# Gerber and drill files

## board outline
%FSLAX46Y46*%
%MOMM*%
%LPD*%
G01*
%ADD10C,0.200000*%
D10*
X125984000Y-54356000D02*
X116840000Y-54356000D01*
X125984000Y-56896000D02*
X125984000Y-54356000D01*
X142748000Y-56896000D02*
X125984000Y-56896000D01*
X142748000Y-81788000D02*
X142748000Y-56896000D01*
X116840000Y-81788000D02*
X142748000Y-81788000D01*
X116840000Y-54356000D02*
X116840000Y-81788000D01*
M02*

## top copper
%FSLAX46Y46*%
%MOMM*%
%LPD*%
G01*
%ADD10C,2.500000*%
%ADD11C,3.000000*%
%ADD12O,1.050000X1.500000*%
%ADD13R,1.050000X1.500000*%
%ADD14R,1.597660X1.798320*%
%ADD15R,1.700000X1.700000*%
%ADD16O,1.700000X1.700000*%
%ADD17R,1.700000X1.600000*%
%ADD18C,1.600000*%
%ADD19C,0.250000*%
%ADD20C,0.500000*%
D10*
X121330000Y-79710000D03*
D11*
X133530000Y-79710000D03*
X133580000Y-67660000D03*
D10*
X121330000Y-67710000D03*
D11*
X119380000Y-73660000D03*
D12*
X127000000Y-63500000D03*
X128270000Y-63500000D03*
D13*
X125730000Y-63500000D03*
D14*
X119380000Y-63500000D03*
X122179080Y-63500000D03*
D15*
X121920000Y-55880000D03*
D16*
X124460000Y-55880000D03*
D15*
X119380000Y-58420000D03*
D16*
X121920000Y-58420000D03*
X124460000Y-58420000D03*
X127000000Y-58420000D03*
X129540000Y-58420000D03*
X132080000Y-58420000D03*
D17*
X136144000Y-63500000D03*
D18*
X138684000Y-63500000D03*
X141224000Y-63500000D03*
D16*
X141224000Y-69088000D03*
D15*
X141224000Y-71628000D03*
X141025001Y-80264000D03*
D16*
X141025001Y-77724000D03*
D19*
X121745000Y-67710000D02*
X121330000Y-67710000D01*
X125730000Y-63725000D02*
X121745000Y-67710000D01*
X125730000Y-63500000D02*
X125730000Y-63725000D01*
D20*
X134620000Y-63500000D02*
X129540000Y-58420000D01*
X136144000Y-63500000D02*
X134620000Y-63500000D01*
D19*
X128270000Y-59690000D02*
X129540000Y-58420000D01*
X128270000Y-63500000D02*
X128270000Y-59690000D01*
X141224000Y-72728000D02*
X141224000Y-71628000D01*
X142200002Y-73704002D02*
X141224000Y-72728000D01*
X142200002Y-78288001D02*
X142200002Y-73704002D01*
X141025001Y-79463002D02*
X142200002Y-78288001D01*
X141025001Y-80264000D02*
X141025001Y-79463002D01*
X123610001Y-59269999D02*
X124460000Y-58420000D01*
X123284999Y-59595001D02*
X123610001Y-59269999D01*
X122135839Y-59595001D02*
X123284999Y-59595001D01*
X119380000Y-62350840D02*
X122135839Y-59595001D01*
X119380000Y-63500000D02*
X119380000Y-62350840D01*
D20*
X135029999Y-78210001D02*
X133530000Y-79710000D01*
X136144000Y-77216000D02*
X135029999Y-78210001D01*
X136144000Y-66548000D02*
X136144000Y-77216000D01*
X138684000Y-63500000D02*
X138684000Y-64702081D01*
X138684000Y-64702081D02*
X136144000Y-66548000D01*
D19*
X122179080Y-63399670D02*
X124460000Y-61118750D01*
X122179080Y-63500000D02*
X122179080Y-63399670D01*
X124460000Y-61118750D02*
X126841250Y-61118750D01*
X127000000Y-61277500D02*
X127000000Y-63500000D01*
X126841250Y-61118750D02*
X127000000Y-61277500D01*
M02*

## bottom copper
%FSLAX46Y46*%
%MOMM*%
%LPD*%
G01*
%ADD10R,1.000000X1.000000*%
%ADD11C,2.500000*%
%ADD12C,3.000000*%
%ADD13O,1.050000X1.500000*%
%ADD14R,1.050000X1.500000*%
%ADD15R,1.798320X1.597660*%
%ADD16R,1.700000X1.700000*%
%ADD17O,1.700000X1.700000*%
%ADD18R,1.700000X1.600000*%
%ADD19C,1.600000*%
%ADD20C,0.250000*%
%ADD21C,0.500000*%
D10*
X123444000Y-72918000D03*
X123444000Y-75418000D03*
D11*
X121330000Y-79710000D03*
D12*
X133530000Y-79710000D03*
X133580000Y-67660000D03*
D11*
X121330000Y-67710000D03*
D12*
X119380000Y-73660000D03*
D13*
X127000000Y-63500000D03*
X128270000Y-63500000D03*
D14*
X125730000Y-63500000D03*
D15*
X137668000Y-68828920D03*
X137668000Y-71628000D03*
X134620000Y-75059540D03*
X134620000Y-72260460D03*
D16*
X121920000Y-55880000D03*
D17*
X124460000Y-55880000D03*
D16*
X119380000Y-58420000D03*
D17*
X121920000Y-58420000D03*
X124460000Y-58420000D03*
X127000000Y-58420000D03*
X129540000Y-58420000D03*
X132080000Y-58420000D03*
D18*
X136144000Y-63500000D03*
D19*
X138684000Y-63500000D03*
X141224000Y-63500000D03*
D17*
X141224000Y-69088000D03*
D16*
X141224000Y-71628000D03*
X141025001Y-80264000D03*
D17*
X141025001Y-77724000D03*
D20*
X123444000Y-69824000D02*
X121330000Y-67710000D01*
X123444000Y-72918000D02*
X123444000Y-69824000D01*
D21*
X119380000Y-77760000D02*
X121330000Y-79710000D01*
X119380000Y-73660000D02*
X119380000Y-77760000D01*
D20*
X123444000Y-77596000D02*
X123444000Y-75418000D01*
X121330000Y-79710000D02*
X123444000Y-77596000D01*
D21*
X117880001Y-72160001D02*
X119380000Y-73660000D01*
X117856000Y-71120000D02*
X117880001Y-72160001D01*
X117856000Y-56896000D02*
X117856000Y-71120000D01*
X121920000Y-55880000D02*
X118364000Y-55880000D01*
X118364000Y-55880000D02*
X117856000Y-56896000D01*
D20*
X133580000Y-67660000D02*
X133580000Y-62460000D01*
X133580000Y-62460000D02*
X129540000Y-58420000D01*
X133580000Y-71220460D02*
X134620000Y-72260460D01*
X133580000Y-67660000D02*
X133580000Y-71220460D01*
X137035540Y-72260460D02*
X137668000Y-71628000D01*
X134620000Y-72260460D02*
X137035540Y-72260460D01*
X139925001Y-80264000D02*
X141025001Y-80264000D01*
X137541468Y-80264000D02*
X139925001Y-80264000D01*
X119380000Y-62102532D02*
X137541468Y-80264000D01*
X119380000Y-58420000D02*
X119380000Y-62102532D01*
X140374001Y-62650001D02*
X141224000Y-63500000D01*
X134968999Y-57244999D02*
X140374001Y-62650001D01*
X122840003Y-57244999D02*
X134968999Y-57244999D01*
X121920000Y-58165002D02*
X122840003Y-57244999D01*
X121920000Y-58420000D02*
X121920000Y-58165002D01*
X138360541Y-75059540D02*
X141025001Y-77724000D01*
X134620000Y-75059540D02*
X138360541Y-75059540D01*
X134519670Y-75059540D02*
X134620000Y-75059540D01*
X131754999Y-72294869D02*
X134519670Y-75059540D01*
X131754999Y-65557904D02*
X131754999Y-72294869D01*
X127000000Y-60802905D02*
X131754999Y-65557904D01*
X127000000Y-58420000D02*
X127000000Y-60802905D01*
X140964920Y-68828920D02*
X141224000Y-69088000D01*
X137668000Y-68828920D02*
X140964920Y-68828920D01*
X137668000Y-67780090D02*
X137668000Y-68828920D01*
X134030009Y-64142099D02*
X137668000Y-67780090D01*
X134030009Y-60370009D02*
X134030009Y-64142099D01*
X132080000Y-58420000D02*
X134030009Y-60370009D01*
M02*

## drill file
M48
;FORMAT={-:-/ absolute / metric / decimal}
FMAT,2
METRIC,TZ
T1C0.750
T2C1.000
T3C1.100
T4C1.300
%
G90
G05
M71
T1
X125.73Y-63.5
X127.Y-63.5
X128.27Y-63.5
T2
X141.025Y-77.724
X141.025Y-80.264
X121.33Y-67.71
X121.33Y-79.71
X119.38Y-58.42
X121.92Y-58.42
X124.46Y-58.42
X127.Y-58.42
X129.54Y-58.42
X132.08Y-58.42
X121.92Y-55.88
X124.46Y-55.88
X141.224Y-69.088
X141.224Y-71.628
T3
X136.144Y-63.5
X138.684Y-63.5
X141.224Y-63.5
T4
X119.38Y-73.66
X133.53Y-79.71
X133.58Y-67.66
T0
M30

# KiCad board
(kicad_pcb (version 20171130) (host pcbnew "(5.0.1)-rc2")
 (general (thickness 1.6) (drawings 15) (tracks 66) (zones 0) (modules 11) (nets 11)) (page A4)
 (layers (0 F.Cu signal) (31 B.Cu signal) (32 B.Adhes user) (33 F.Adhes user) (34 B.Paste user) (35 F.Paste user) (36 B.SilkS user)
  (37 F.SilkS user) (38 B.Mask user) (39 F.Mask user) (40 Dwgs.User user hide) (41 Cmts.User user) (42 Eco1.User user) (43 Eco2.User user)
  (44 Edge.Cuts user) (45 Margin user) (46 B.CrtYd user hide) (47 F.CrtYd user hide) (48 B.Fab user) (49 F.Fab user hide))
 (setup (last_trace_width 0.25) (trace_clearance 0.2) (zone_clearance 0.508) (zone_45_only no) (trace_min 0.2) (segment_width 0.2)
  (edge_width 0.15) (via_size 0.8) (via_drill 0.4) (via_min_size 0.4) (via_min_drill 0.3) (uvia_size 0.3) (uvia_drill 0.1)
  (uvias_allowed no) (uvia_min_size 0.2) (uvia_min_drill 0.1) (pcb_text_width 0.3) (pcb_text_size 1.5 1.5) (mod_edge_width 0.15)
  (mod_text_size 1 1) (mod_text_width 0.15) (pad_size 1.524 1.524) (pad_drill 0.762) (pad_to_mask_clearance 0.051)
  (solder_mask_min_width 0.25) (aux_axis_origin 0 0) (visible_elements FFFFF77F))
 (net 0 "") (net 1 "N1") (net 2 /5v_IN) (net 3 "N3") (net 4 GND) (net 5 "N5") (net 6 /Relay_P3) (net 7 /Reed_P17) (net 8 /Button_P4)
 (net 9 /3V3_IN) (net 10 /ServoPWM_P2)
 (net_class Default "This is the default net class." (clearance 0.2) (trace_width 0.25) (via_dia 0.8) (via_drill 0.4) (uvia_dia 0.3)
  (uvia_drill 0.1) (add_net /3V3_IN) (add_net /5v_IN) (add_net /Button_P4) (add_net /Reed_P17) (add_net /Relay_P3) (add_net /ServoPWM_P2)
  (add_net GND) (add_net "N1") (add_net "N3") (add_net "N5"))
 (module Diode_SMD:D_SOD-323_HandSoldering (layer B.Cu) (at 123.444 74.168 270)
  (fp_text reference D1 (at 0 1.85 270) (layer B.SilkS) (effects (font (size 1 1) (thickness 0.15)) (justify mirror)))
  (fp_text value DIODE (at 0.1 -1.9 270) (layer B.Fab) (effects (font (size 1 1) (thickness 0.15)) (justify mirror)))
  (pad 1 smd rect (at -1.25 0 270) (size 1 1) (layers B.Cu B.Paste B.Mask) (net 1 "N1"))
  (pad 2 smd rect (at 1.25 0 270) (size 1 1) (layers B.Cu B.Paste B.Mask) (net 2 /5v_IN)))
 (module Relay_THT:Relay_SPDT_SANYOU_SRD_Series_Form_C (layer F.Cu) (at 119.38 73.66)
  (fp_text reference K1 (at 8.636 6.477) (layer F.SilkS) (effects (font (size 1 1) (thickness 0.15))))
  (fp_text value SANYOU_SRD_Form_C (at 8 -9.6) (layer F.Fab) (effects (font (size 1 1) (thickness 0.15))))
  (pad 2 thru_hole circle (at 1.95 6.05 90) (size 2.5 2.5) (drill 1) (layers *.Cu *.Mask) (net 2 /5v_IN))
  (pad 3 thru_hole circle (at 14.15 6.05 90) (size 3 3) (drill 1.3) (layers *.Cu *.Mask) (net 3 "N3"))
  (pad 4 thru_hole circle (at 14.2 -6 90) (size 3 3) (drill 1.3) (layers *.Cu *.Mask) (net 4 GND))
  (pad 5 thru_hole circle (at 1.95 -5.95 90) (size 2.5 2.5) (drill 1) (layers *.Cu *.Mask) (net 1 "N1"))
  (pad 1 thru_hole circle (at 0 0 90) (size 3 3) (drill 1.3) (layers *.Cu *.Mask) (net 2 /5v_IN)))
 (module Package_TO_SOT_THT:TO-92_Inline (layer F.Cu) (at 125.73 63.5)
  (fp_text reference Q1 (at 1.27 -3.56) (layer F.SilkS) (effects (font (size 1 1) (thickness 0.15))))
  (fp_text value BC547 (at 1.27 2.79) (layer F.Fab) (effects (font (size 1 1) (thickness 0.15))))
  (pad 2 thru_hole oval (at 1.27 0) (size 1.05 1.5) (drill 0.75) (layers *.Cu *.Mask) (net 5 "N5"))
  (pad 3 thru_hole oval (at 2.54 0) (size 1.05 1.5) (drill 0.75) (layers *.Cu *.Mask) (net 4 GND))
  (pad 1 thru_hole rect (at 0 0) (size 1.05 1.5) (drill 0.75) (layers *.Cu *.Mask) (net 1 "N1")))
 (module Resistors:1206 (layer F.Cu) (at 120.77954 63.5 180)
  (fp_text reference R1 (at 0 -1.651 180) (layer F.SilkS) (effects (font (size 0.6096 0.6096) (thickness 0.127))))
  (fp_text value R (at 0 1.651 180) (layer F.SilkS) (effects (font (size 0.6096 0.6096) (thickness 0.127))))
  (pad 2 smd rect (at 1.39954 0 180) (size 1.59766 1.79832) (layers F.Cu F.Paste F.Mask) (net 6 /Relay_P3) (solder_mask_margin 0.1016))
  (pad 1 smd rect (at -1.39954 0 180) (size 1.59766 1.79832) (layers F.Cu F.Paste F.Mask) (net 5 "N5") (solder_mask_margin 0.1016)))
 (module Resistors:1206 (layer B.Cu) (at 137.668 70.22846 270)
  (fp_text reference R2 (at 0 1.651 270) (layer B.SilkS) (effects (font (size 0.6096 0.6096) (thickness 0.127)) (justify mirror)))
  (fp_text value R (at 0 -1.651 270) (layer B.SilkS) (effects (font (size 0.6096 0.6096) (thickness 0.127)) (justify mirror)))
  (pad 1 smd rect (at -1.39954 0 270) (size 1.59766 1.79832) (layers B.Cu B.Paste B.Mask) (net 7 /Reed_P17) (solder_mask_margin 0.1016))
  (pad 2 smd rect (at 1.39954 0 270) (size 1.59766 1.79832) (layers B.Cu B.Paste B.Mask) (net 4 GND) (solder_mask_margin 0.1016)))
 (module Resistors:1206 (layer B.Cu) (at 134.62 73.66 90)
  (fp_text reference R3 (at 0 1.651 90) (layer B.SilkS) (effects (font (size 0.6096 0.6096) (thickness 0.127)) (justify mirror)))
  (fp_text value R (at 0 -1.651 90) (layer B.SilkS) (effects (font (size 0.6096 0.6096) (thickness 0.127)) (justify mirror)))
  (pad 1 smd rect (at -1.39954 0 90) (size 1.59766 1.79832) (layers B.Cu B.Paste B.Mask) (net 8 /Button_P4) (solder_mask_margin 0.1016))
  (pad 2 smd rect (at 1.39954 0 90) (size 1.59766 1.79832) (layers B.Cu B.Paste B.Mask) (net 4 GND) (solder_mask_margin 0.1016)))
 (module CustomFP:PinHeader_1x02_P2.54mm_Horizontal (layer F.Cu) (at 121.92 55.88 90)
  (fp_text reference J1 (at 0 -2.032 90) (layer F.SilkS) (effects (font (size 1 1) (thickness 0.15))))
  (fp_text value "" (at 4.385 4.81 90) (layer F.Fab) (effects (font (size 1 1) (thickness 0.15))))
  (pad 1 thru_hole rect (at 0 0 90) (size 1.7 1.7) (drill 1) (layers *.Cu *.Mask) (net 2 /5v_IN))
  (pad 2 thru_hole oval (at 0 2.54 90) (size 1.7 1.7) (drill 1) (layers *.Cu *.Mask)))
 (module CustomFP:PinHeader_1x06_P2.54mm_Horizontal (layer F.Cu) (at 119.38 58.42 90)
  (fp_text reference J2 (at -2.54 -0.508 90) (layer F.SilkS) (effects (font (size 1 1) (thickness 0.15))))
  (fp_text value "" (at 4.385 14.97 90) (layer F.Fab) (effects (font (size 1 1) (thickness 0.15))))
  (pad 1 thru_hole rect (at 0 0 90) (size 1.7 1.7) (drill 1) (layers *.Cu *.Mask) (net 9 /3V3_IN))
  (pad 2 thru_hole oval (at 0 2.54 90) (size 1.7 1.7) (drill 1) (layers *.Cu *.Mask) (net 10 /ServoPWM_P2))
  (pad 3 thru_hole oval (at 0 5.08 90) (size 1.7 1.7) (drill 1) (layers *.Cu *.Mask) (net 6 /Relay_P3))
  (pad 4 thru_hole oval (at 0 7.62 90) (size 1.7 1.7) (drill 1) (layers *.Cu *.Mask) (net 8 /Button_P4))
  (pad 5 thru_hole oval (at 0 10.16 90) (size 1.7 1.7) (drill 1) (layers *.Cu *.Mask) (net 4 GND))
  (pad 6 thru_hole oval (at 0 12.7 90) (size 1.7 1.7) (drill 1) (layers *.Cu *.Mask) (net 7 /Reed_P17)))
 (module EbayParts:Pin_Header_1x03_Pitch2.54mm (layer F.Cu) (at 136.144 63.5 90)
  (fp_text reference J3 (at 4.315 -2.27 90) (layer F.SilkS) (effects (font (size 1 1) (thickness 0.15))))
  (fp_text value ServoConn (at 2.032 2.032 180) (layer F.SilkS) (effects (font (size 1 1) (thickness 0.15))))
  (pad 1 thru_hole rect (at 0 0 90) (size 1.6 1.7) (drill 1.1) (layers *.Cu *.Mask) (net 4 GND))
  (pad 2 thru_hole circle (at 0 2.54 90) (size 1.6 1.6) (drill 1.1) (layers *.Cu *.Mask) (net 3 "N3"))
  (pad 3 thru_hole circle (at 0 5.08 90) (size 1.6 1.6) (drill 1.1) (layers *.Cu *.Mask) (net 10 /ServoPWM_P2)))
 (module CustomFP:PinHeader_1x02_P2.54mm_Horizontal (layer F.Cu) (at 141.224 71.628 180)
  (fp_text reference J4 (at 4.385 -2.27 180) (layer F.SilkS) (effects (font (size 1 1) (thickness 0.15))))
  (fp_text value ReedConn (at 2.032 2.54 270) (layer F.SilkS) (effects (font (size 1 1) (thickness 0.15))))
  (pad 2 thru_hole oval (at 0 2.54 180) (size 1.7 1.7) (drill 1) (layers *.Cu *.Mask) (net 7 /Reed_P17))
  (pad 1 thru_hole rect (at 0 0 180) (size 1.7 1.7) (drill 1) (layers *.Cu *.Mask) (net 9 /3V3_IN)))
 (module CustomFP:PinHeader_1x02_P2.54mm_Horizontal (layer F.Cu) (at 141.025001 80.264 180)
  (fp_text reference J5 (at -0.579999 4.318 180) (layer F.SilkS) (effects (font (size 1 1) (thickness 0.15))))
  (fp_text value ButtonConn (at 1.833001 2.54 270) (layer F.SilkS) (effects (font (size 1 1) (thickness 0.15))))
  (pad 1 thru_hole rect (at 0 0 180) (size 1.7 1.7) (drill 1) (layers *.Cu *.Mask) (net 9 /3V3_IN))
  (pad 2 thru_hole oval (at 0 2.54 180) (size 1.7 1.7) (drill 1) (layers *.Cu *.Mask) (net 8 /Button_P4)))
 (gr_line (start 125.984 54.356) (end 116.84 54.356) (layer Edge.Cuts) (width 0.2))
 (gr_line (start 125.984 56.896) (end 125.984 54.356) (layer Edge.Cuts) (width 0.2))
 (gr_line (start 142.748 56.896) (end 125.984 56.896) (layer Edge.Cuts) (width 0.2))
 (gr_line (start 142.748 81.788) (end 142.748 56.896) (layer Edge.Cuts) (width 0.2))
 (gr_line (start 116.84 81.788) (end 142.748 81.788) (layer Edge.Cuts) (width 0.2))
 (gr_line (start 116.84 54.356) (end 116.84 81.788) (layer Edge.Cuts) (width 0.2))
 (segment (start 121.745 67.71) (end 121.33 67.71) (width 0.25) (layer F.Cu) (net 1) (status 30))
 (segment (start 125.73 63.725) (end 121.745 67.71) (width 0.25) (layer F.Cu) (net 1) (status 30))
 (segment (start 125.73 63.5) (end 125.73 63.725) (width 0.25) (layer F.Cu) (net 1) (status 30))
 (segment (start 123.444 69.824) (end 121.33 67.71) (width 0.25) (layer B.Cu) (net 1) (status 20))
 (segment (start 123.444 72.918) (end 123.444 69.824) (width 0.25) (layer B.Cu) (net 1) (status 10))
 (segment (start 119.38 77.76) (end 121.33 79.71) (width 0.5) (layer B.Cu) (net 2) (status 20))
 (segment (start 119.38 73.66) (end 119.38 77.76) (width 0.5) (layer B.Cu) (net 2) (status 10))
 (segment (start 123.444 77.596) (end 123.444 75.418) (width 0.25) (layer B.Cu) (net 2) (status 20))
 (segment (start 121.33 79.71) (end 123.444 77.596) (width 0.25) (layer B.Cu) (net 2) (status 10))
 (segment (start 117.880001 72.160001) (end 119.38 73.66) (width 0.5) (layer B.Cu) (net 2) (status 20))
 (segment (start 117.856 71.12) (end 117.880001 72.160001) (width 0.5) (layer B.Cu) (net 2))
 (segment (start 117.856 56.896) (end 117.856 71.12) (width 0.5) (layer B.Cu) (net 2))
 (segment (start 121.92 55.88) (end 118.364 55.88) (width 0.5) (layer B.Cu) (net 2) (status 10))
 (segment (start 118.364 55.88) (end 117.856 56.896) (width 0.5) (layer B.Cu) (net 2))
 (segment (start 133.58 67.66) (end 133.58 62.46) (width 0.25) (layer B.Cu) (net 4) (status 10))
 (segment (start 133.58 62.46) (end 129.54 58.42) (width 0.25) (layer B.Cu) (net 4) (status 20))
 (segment (start 133.58 71.22046) (end 134.62 72.26046) (width 0.25) (layer B.Cu) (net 4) (status 20))
 (segment (start 133.58 67.66) (end 133.58 71.22046) (width 0.25) (layer B.Cu) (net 4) (status 10))
 (segment (start 137.03554 72.26046) (end 137.668 71.628) (width 0.25) (layer B.Cu) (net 4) (status 30))
 (segment (start 134.62 72.26046) (end 137.03554 72.26046) (width 0.25) (layer B.Cu) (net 4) (status 30))
 (segment (start 134.62 63.5) (end 129.54 58.42) (width 0.5) (layer F.Cu) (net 4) (status 20))
 (segment (start 136.144 63.5) (end 134.62 63.5) (width 0.5) (layer F.Cu) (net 4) (status 10))
 (segment (start 128.27 59.69) (end 129.54 58.42) (width 0.25) (layer F.Cu) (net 4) (status 20))
 (segment (start 128.27 63.5) (end 128.27 59.69) (width 0.25) (layer F.Cu) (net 4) (status 10))
 (segment (start 139.925001 80.264) (end 141.025001 80.264) (width 0.25) (layer B.Cu) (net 9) (status 20))
 (segment (start 137.541468 80.264) (end 139.925001 80.264) (width 0.25) (layer B.Cu) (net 9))
 (segment (start 119.38 62.102532) (end 137.541468 80.264) (width 0.25) (layer B.Cu) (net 9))
 (segment (start 119.38 58.42) (end 119.38 62.102532) (width 0.25) (layer B.Cu) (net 9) (status 10))
 (segment (start 141.224 72.728) (end 141.224 71.628) (width 0.25) (layer F.Cu) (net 9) (status 20))
 (segment (start 142.200002 73.704002) (end 141.224 72.728) (width 0.25) (layer F.Cu) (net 9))
 (segment (start 142.200002 78.288001) (end 142.200002 73.704002) (width 0.25) (layer F.Cu) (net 9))
 (segment (start 141.025001 79.463002) (end 142.200002 78.288001) (width 0.25) (layer F.Cu) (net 9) (status 10))
 (segment (start 141.025001 80.264) (end 141.025001 79.463002) (width 0.25) (layer F.Cu) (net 9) (status 30))
 (segment (start 140.374001 62.650001) (end 141.224 63.5) (width 0.25) (layer B.Cu) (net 10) (status 20))
 (segment (start 134.968999 57.244999) (end 140.374001 62.650001) (width 0.25) (layer B.Cu) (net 10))
 (segment (start 122.840003 57.244999) (end 134.968999 57.244999) (width 0.25) (layer B.Cu) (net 10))
 (segment (start 121.92 58.165002) (end 122.840003 57.244999) (width 0.25) (layer B.Cu) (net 10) (status 10))
 (segment (start 121.92 58.42) (end 121.92 58.165002) (width 0.25) (layer B.Cu) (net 10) (status 30))
 (segment (start 123.610001 59.269999) (end 124.46 58.42) (width 0.25) (layer F.Cu) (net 6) (status 30))
 (segment (start 123.284999 59.595001) (end 123.610001 59.269999) (width 0.25) (layer F.Cu) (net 6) (status 20))
 (segment (start 122.135839 59.595001) (end 123.284999 59.595001) (width 0.25) (layer F.Cu) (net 6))
 (segment (start 119.38 62.35084) (end 122.135839 59.595001) (width 0.25) (layer F.Cu) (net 6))
 (segment (start 119.38 63.5) (end 119.38 62.35084) (width 0.25) (layer F.Cu) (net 6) (status 10))
 (segment (start 138.360541 75.05954) (end 141.025001 77.724) (width 0.25) (layer B.Cu) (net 8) (status 20))
 (segment (start 134.62 75.05954) (end 138.360541 75.05954) (width 0.25) (layer B.Cu) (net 8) (status 10))
 (segment (start 134.51967 75.05954) (end 134.62 75.05954) (width 0.25) (layer B.Cu) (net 8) (status 30))
 (segment (start 131.754999 72.294869) (end 134.51967 75.05954) (width 0.25) (layer B.Cu) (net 8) (status 20))
 (segment (start 131.754999 65.557904) (end 131.754999 72.294869) (width 0.25) (layer B.Cu) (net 8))
 (segment (start 127 60.802905) (end 131.754999 65.557904) (width 0.25) (layer B.Cu) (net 8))
 (segment (start 127 58.42) (end 127 60.802905) (width 0.25) (layer B.Cu) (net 8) (status 10))
 (segment (start 140.96492 68.82892) (end 141.224 69.088) (width 0.25) (layer B.Cu) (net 7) (status 30))
 (segment (start 137.668 68.82892) (end 140.96492 68.82892) (width 0.25) (layer B.Cu) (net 7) (status 30))
 (segment (start 137.668 67.78009) (end 137.668 68.82892) (width 0.25) (layer B.Cu) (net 7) (status 20))
 (segment (start 134.030009 64.142099) (end 137.668 67.78009) (width 0.25) (layer B.Cu) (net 7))
 (segment (start 134.030009 60.370009) (end 134.030009 64.142099) (width 0.25) (layer B.Cu) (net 7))
 (segment (start 132.08 58.42) (end 134.030009 60.370009) (width 0.25) (layer B.Cu) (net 7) (status 10))
 (segment (start 135.029999 78.210001) (end 133.53 79.71) (width 0.5) (layer F.Cu) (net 3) (status 20))
 (segment (start 136.144 77.216) (end 135.029999 78.210001) (width 0.5) (layer F.Cu) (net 3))
 (segment (start 136.144 66.548) (end 136.144 77.216) (width 0.5) (layer F.Cu) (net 3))
 (segment (start 138.684 63.5) (end 138.684 64.702081) (width 0.5) (layer F.Cu) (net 3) (status 10))
 (segment (start 138.684 64.702081) (end 136.144 66.548) (width 0.5) (layer F.Cu) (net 3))
 (segment (start 122.17908 63.39967) (end 124.46 61.11875) (width 0.25) (layer F.Cu) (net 5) (status 10))
 (segment (start 122.17908 63.5) (end 122.17908 63.39967) (width 0.25) (layer F.Cu) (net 5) (status 30))
 (segment (start 124.46 61.11875) (end 126.84125 61.11875) (width 0.25) (layer F.Cu) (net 5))
 (segment (start 127 61.2775) (end 127 63.5) (width 0.25) (layer F.Cu) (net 5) (status 20))
 (segment (start 126.84125 61.11875) (end 127 61.2775) (width 0.25) (layer F.Cu) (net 5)))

